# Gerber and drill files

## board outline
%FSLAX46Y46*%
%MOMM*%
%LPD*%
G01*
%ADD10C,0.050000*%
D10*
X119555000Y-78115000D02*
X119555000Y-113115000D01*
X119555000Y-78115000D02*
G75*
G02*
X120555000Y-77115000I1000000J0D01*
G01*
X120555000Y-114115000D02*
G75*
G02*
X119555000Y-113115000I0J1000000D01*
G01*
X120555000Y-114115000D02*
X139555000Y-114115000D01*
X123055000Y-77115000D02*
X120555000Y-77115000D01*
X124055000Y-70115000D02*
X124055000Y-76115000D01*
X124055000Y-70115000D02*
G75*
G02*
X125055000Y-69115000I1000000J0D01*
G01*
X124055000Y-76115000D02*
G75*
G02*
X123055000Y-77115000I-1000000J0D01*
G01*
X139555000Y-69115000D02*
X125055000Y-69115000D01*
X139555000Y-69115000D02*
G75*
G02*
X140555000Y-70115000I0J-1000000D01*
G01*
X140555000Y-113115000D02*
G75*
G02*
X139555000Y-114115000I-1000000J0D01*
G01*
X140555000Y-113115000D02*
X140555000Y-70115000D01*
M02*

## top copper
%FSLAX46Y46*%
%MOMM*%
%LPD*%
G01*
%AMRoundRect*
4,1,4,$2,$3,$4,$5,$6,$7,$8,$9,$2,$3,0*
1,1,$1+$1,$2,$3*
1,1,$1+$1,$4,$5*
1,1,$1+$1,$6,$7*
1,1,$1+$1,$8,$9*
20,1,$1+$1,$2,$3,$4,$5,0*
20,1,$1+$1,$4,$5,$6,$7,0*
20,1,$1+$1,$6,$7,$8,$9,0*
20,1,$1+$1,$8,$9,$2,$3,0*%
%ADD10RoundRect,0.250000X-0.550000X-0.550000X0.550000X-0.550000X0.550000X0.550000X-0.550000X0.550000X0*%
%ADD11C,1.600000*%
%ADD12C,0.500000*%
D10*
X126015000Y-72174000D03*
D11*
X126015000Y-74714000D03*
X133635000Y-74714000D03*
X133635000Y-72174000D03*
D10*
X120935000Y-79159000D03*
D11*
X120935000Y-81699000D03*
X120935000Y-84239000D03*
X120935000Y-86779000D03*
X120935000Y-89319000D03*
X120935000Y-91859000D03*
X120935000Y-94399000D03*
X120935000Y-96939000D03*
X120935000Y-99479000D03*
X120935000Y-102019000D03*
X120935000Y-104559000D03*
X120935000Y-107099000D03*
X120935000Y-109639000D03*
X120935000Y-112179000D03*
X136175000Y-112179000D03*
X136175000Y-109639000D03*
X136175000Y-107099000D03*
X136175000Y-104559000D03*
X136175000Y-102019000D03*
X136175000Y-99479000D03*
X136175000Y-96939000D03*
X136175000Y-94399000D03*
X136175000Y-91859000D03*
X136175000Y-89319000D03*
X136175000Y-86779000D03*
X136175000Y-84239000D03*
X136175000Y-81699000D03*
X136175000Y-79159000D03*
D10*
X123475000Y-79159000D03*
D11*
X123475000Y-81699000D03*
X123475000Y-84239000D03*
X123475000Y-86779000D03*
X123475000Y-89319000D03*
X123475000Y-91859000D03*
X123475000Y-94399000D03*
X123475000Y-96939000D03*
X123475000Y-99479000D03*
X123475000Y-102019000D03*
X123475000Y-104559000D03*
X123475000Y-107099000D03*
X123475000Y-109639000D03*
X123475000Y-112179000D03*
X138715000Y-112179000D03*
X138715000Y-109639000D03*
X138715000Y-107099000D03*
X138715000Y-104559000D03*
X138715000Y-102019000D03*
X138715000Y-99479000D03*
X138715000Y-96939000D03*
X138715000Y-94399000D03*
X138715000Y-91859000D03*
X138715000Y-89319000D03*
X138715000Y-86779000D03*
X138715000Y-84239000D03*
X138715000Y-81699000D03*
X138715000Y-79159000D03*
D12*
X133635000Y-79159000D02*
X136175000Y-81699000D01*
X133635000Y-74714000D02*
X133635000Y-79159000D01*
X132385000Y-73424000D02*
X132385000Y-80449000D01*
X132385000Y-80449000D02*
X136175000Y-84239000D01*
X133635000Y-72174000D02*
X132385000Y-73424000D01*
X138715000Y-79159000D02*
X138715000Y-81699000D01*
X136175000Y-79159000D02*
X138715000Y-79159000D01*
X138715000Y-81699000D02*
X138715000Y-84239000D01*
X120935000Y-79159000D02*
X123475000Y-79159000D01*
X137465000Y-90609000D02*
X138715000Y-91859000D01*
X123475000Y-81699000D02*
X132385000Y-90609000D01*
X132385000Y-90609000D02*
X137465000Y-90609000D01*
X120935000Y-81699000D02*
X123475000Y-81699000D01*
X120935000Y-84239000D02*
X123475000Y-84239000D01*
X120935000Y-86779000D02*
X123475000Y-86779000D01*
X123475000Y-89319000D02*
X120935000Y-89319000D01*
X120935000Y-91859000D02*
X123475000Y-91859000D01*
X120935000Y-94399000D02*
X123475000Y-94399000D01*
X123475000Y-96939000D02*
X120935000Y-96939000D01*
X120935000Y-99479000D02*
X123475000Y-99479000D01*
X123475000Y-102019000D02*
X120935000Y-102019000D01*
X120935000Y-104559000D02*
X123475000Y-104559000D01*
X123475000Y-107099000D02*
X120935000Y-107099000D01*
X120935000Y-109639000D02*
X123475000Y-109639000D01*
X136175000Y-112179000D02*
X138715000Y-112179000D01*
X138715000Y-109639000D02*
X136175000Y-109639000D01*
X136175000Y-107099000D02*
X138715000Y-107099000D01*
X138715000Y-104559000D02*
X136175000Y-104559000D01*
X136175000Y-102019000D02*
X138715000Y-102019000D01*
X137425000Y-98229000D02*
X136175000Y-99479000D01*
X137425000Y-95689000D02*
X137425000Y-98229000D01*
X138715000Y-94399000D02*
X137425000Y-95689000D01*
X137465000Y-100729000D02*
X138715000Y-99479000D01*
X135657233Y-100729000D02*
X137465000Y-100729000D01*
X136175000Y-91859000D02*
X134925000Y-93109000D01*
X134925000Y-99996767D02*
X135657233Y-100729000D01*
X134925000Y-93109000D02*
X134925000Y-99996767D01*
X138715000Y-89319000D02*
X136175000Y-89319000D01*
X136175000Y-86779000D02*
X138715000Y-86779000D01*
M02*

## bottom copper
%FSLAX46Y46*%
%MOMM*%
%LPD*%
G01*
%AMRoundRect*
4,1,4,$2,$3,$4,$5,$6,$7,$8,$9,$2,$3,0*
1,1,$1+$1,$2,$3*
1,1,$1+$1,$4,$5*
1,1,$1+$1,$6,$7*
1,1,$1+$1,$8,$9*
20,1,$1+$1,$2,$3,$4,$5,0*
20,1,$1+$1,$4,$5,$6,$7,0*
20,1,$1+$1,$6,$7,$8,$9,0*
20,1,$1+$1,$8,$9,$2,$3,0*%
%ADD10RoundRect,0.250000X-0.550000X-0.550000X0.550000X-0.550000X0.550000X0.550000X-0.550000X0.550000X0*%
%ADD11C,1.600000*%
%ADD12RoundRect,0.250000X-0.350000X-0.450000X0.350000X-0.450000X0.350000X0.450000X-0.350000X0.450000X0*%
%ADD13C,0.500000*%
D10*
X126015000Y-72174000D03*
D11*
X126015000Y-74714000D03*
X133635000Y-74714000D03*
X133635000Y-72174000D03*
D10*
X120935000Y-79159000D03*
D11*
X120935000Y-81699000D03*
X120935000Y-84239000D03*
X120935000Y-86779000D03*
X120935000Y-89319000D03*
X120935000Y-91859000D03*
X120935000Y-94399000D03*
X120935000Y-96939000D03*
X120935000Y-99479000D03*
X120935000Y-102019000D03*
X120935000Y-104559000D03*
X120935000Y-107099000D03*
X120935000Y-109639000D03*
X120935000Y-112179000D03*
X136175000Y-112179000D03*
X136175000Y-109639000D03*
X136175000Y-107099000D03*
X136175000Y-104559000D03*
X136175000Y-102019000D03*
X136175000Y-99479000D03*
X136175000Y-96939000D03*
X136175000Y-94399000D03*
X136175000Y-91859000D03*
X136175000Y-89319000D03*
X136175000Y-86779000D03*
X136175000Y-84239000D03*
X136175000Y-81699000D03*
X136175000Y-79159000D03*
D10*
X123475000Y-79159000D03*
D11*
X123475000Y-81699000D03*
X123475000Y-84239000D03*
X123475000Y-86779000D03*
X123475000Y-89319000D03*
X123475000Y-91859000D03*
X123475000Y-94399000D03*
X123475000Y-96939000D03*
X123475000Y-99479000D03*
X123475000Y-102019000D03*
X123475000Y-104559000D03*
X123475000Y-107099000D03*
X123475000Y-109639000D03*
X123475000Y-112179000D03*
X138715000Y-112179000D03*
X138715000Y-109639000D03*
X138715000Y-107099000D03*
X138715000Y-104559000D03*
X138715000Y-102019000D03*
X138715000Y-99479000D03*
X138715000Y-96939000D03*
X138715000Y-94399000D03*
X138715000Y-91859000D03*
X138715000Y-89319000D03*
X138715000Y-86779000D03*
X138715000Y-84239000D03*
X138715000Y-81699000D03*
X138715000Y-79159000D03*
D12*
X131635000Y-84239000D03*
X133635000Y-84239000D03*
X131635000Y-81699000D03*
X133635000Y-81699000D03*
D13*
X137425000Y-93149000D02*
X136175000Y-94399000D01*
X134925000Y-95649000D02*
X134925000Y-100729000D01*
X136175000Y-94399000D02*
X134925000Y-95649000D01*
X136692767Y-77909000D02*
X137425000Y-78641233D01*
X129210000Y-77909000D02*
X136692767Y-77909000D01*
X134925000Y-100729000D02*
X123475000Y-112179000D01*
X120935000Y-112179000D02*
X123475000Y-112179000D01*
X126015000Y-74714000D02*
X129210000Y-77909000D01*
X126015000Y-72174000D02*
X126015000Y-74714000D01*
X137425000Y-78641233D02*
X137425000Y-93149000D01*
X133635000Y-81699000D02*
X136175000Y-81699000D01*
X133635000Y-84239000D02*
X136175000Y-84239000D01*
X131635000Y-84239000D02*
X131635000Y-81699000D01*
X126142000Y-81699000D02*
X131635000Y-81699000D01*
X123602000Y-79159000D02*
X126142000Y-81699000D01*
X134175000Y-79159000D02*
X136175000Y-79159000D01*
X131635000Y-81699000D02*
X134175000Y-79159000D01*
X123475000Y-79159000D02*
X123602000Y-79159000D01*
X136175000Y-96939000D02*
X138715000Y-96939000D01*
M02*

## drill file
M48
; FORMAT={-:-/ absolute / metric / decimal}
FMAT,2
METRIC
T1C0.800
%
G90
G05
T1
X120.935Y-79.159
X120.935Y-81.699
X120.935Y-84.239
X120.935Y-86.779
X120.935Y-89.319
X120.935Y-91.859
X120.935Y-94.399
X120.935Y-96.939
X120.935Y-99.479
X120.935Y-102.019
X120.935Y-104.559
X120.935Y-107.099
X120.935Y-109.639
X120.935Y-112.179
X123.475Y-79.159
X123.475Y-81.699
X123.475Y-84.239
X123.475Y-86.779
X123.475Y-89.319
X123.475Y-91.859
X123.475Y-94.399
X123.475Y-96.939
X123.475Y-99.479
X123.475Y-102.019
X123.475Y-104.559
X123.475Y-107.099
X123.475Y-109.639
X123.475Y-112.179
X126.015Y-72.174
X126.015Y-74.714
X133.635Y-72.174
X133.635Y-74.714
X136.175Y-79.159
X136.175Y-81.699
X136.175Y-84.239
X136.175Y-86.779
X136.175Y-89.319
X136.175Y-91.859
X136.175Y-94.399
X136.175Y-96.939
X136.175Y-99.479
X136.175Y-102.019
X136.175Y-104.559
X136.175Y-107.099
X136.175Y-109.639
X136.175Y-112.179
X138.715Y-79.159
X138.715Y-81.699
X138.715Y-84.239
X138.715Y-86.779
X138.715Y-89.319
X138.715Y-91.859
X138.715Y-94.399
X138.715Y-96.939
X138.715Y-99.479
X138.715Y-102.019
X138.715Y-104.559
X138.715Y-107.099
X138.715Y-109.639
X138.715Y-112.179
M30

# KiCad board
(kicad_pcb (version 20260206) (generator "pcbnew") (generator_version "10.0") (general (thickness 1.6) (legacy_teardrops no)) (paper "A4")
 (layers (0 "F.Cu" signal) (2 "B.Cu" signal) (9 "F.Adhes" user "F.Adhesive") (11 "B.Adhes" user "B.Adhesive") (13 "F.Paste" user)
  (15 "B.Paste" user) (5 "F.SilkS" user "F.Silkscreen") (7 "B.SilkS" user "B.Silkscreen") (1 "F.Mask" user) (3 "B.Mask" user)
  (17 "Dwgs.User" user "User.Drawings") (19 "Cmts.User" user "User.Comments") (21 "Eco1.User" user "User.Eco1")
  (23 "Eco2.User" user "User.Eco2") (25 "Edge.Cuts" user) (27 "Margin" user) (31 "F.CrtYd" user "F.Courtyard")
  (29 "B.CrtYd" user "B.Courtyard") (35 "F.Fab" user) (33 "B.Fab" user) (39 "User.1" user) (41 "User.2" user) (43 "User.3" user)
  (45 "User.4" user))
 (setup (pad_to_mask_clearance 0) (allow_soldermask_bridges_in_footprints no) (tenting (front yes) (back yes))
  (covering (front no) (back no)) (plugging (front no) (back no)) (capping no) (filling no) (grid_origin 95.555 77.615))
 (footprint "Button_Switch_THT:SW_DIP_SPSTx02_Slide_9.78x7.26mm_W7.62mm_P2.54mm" (layer "F.Cu") (at 126.015 72.174)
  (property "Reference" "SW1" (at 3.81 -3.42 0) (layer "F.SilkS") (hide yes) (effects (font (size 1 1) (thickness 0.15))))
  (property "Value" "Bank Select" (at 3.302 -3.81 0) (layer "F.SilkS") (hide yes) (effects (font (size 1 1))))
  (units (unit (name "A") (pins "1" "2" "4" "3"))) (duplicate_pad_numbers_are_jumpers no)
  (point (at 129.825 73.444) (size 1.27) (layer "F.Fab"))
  (pad "1" thru_hole roundrect (at 0 0) (size 1.6 1.6) (drill 0.8) (layers "*.Cu" "*.Mask") (remove_unused_layers no)
   (roundrect_rratio 0.15625) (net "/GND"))
  (pad "2" thru_hole circle (at 0 2.54) (size 1.6 1.6) (drill 0.8) (layers "*.Cu" "*.Mask") (remove_unused_layers no) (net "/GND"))
  (pad "3" thru_hole circle (at 7.62 2.54) (size 1.6 1.6) (drill 0.8) (layers "*.Cu" "*.Mask") (remove_unused_layers no) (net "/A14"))
  (pad "4" thru_hole circle (at 7.62 0) (size 1.6 1.6) (drill 0.8) (layers "*.Cu" "*.Mask") (remove_unused_layers no) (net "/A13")))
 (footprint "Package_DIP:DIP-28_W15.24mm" (layer "F.Cu") (at 120.935 79.159)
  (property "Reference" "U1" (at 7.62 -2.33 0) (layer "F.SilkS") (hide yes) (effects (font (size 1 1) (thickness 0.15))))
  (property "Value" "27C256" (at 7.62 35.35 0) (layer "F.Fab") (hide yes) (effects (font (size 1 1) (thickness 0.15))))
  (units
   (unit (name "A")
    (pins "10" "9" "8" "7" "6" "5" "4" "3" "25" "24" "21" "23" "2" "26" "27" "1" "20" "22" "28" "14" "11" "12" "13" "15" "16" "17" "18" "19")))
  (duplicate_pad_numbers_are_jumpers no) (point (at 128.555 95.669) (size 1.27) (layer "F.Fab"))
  (pad "1" thru_hole roundrect (at 0 0) (size 1.6 1.6) (drill 0.8) (layers "*.Cu" "*.Mask") (remove_unused_layers no)
   (roundrect_rratio 0.15625) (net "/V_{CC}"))
  (pad "2" thru_hole circle (at 0 2.54) (size 1.6 1.6) (drill 0.8) (layers "*.Cu" "*.Mask") (remove_unused_layers no) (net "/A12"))
  (pad "3" thru_hole circle (at 0 5.08) (size 1.6 1.6) (drill 0.8) (layers "*.Cu" "*.Mask") (remove_unused_layers no) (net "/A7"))
  (pad "4" thru_hole circle (at 0 7.62) (size 1.6 1.6) (drill 0.8) (layers "*.Cu" "*.Mask") (remove_unused_layers no) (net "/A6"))
  (pad "5" thru_hole circle (at 0 10.16) (size 1.6 1.6) (drill 0.8) (layers "*.Cu" "*.Mask") (remove_unused_layers no) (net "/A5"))
  (pad "6" thru_hole circle (at 0 12.7) (size 1.6 1.6) (drill 0.8) (layers "*.Cu" "*.Mask") (remove_unused_layers no) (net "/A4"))
  (pad "7" thru_hole circle (at 0 15.24) (size 1.6 1.6) (drill 0.8) (layers "*.Cu" "*.Mask") (remove_unused_layers no) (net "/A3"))
  (pad "8" thru_hole circle (at 0 17.78) (size 1.6 1.6) (drill 0.8) (layers "*.Cu" "*.Mask") (remove_unused_layers no) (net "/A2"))
  (pad "9" thru_hole circle (at 0 20.32) (size 1.6 1.6) (drill 0.8) (layers "*.Cu" "*.Mask") (remove_unused_layers no) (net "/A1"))
  (pad "10" thru_hole circle (at 0 22.86) (size 1.6 1.6) (drill 0.8) (layers "*.Cu" "*.Mask") (remove_unused_layers no) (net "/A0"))
  (pad "11" thru_hole circle (at 0 25.4) (size 1.6 1.6) (drill 0.8) (layers "*.Cu" "*.Mask") (remove_unused_layers no) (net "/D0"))
  (pad "12" thru_hole circle (at 0 27.94) (size 1.6 1.6) (drill 0.8) (layers "*.Cu" "*.Mask") (remove_unused_layers no) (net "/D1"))
  (pad "13" thru_hole circle (at 0 30.48) (size 1.6 1.6) (drill 0.8) (layers "*.Cu" "*.Mask") (remove_unused_layers no) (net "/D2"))
  (pad "14" thru_hole circle (at 0 33.02) (size 1.6 1.6) (drill 0.8) (layers "*.Cu" "*.Mask") (remove_unused_layers no) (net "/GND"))
  (pad "15" thru_hole circle (at 15.24 33.02) (size 1.6 1.6) (drill 0.8) (layers "*.Cu" "*.Mask") (remove_unused_layers no) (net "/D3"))
  (pad "16" thru_hole circle (at 15.24 30.48) (size 1.6 1.6) (drill 0.8) (layers "*.Cu" "*.Mask") (remove_unused_layers no) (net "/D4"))
  (pad "17" thru_hole circle (at 15.24 27.94) (size 1.6 1.6) (drill 0.8) (layers "*.Cu" "*.Mask") (remove_unused_layers no) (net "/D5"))
  (pad "18" thru_hole circle (at 15.24 25.4) (size 1.6 1.6) (drill 0.8) (layers "*.Cu" "*.Mask") (remove_unused_layers no) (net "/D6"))
  (pad "19" thru_hole circle (at 15.24 22.86) (size 1.6 1.6) (drill 0.8) (layers "*.Cu" "*.Mask") (remove_unused_layers no) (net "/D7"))
  (pad "20" thru_hole circle (at 15.24 20.32) (size 1.6 1.6) (drill 0.8) (layers "*.Cu" "*.Mask") (remove_unused_layers no) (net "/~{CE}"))
  (pad "21" thru_hole circle (at 15.24 17.78) (size 1.6 1.6) (drill 0.8) (layers "*.Cu" "*.Mask") (remove_unused_layers no) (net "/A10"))
  (pad "22" thru_hole circle (at 15.24 15.24) (size 1.6 1.6) (drill 0.8) (layers "*.Cu" "*.Mask") (remove_unused_layers no) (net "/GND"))
  (pad "23" thru_hole circle (at 15.24 12.7) (size 1.6 1.6) (drill 0.8) (layers "*.Cu" "*.Mask") (remove_unused_layers no) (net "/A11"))
  (pad "24" thru_hole circle (at 15.24 10.16) (size 1.6 1.6) (drill 0.8) (layers "*.Cu" "*.Mask") (remove_unused_layers no) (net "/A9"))
  (pad "25" thru_hole circle (at 15.24 7.62) (size 1.6 1.6) (drill 0.8) (layers "*.Cu" "*.Mask") (remove_unused_layers no) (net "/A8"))
  (pad "26" thru_hole circle (at 15.24 5.08) (size 1.6 1.6) (drill 0.8) (layers "*.Cu" "*.Mask") (remove_unused_layers no) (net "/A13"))
  (pad "27" thru_hole circle (at 15.24 2.54) (size 1.6 1.6) (drill 0.8) (layers "*.Cu" "*.Mask") (remove_unused_layers no) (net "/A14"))
  (pad "28" thru_hole circle (at 15.24 0) (size 1.6 1.6) (drill 0.8) (layers "*.Cu" "*.Mask") (remove_unused_layers no) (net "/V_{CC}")))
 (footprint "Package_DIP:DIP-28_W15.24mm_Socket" (layer "F.Cu") (at 123.475 79.159)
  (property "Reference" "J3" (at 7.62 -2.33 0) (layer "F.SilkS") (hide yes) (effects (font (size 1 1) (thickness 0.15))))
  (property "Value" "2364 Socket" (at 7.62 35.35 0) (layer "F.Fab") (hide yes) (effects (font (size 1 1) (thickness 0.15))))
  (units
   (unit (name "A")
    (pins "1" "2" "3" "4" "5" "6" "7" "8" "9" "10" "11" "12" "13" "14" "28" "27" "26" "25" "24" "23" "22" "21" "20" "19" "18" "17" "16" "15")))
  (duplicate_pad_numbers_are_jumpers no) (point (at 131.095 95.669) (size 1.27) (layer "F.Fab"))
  (pad "1" thru_hole roundrect (at 0 0) (size 1.6 1.6) (drill 0.8) (layers "*.Cu" "*.Mask") (remove_unused_layers no)
   (roundrect_rratio 0.15625) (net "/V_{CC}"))
  (pad "2" thru_hole circle (at 0 2.54) (size 1.6 1.6) (drill 0.8) (layers "*.Cu" "*.Mask") (remove_unused_layers no) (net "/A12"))
  (pad "3" thru_hole circle (at 0 5.08) (size 1.6 1.6) (drill 0.8) (layers "*.Cu" "*.Mask") (remove_unused_layers no) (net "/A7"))
  (pad "4" thru_hole circle (at 0 7.62) (size 1.6 1.6) (drill 0.8) (layers "*.Cu" "*.Mask") (remove_unused_layers no) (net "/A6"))
  (pad "5" thru_hole circle (at 0 10.16) (size 1.6 1.6) (drill 0.8) (layers "*.Cu" "*.Mask") (remove_unused_layers no) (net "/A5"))
  (pad "6" thru_hole circle (at 0 12.7) (size 1.6 1.6) (drill 0.8) (layers "*.Cu" "*.Mask") (remove_unused_layers no) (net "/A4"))
  (pad "7" thru_hole circle (at 0 15.24) (size 1.6 1.6) (drill 0.8) (layers "*.Cu" "*.Mask") (remove_unused_layers no) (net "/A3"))
  (pad "8" thru_hole circle (at 0 17.78) (size 1.6 1.6) (drill 0.8) (layers "*.Cu" "*.Mask") (remove_unused_layers no) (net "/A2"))
  (pad "9" thru_hole circle (at 0 20.32) (size 1.6 1.6) (drill 0.8) (layers "*.Cu" "*.Mask") (remove_unused_layers no) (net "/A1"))
  (pad "10" thru_hole circle (at 0 22.86) (size 1.6 1.6) (drill 0.8) (layers "*.Cu" "*.Mask") (remove_unused_layers no) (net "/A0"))
  (pad "11" thru_hole circle (at 0 25.4) (size 1.6 1.6) (drill 0.8) (layers "*.Cu" "*.Mask") (remove_unused_layers no) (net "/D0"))
  (pad "12" thru_hole circle (at 0 27.94) (size 1.6 1.6) (drill 0.8) (layers "*.Cu" "*.Mask") (remove_unused_layers no) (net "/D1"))
  (pad "13" thru_hole circle (at 0 30.48) (size 1.6 1.6) (drill 0.8) (layers "*.Cu" "*.Mask") (remove_unused_layers no) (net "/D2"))
  (pad "14" thru_hole circle (at 0 33.02) (size 1.6 1.6) (drill 0.8) (layers "*.Cu" "*.Mask") (remove_unused_layers no) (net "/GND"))
  (pad "15" thru_hole circle (at 15.24 33.02) (size 1.6 1.6) (drill 0.8) (layers "*.Cu" "*.Mask") (remove_unused_layers no) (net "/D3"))
  (pad "16" thru_hole circle (at 15.24 30.48) (size 1.6 1.6) (drill 0.8) (layers "*.Cu" "*.Mask") (remove_unused_layers no) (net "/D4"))
  (pad "17" thru_hole circle (at 15.24 27.94) (size 1.6 1.6) (drill 0.8) (layers "*.Cu" "*.Mask") (remove_unused_layers no) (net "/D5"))
  (pad "18" thru_hole circle (at 15.24 25.4) (size 1.6 1.6) (drill 0.8) (layers "*.Cu" "*.Mask") (remove_unused_layers no) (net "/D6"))
  (pad "19" thru_hole circle (at 15.24 22.86) (size 1.6 1.6) (drill 0.8) (layers "*.Cu" "*.Mask") (remove_unused_layers no) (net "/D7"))
  (pad "20" thru_hole circle (at 15.24 20.32) (size 1.6 1.6) (drill 0.8) (layers "*.Cu" "*.Mask") (remove_unused_layers no) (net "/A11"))
  (pad "21" thru_hole circle (at 15.24 17.78) (size 1.6 1.6) (drill 0.8) (layers "*.Cu" "*.Mask") (remove_unused_layers no) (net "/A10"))
  (pad "22" thru_hole circle (at 15.24 15.24) (size 1.6 1.6) (drill 0.8) (layers "*.Cu" "*.Mask") (remove_unused_layers no) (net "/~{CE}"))
  (pad "23" thru_hole circle (at 15.24 12.7) (size 1.6 1.6) (drill 0.8) (layers "*.Cu" "*.Mask") (remove_unused_layers no) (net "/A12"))
  (pad "24" thru_hole circle (at 15.24 10.16) (size 1.6 1.6) (drill 0.8) (layers "*.Cu" "*.Mask") (remove_unused_layers no) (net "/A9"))
  (pad "25" thru_hole circle (at 15.24 7.62) (size 1.6 1.6) (drill 0.8) (layers "*.Cu" "*.Mask") (remove_unused_layers no) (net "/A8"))
  (pad "26" thru_hole circle (at 15.24 5.08) (size 1.6 1.6) (drill 0.8) (layers "*.Cu" "*.Mask") (remove_unused_layers no) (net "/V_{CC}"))
  (pad "27" thru_hole circle (at 15.24 2.54) (size 1.6 1.6) (drill 0.8) (layers "*.Cu" "*.Mask") (remove_unused_layers no) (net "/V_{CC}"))
  (pad "28" thru_hole circle (at 15.24 0) (size 1.6 1.6) (drill 0.8) (layers "*.Cu" "*.Mask") (remove_unused_layers no) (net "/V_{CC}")))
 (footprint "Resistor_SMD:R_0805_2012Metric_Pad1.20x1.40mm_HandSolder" (layer "B.Cu") (at 132.635 84.239)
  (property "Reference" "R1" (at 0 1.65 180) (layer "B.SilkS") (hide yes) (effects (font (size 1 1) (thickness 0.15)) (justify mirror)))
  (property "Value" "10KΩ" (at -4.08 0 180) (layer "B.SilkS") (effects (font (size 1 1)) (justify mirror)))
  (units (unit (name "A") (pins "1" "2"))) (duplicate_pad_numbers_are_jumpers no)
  (pad "1" smd roundrect (at -1 0) (size 1.2 1.4) (layers "B.Cu" "B.Mask" "B.Paste") (roundrect_rratio 0.208333) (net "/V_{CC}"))
  (pad "2" smd roundrect (at 1 0) (size 1.2 1.4) (layers "B.Cu" "B.Mask" "B.Paste") (roundrect_rratio 0.208333) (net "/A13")))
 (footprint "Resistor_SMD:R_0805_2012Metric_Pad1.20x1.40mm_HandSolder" (layer "B.Cu") (at 132.635 81.699)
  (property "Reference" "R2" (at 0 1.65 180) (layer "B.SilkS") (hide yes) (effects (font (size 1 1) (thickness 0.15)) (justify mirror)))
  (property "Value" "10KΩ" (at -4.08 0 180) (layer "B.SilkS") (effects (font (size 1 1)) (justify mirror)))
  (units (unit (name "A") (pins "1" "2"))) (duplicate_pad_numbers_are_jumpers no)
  (pad "1" smd roundrect (at -1 0) (size 1.2 1.4) (layers "B.Cu" "B.Mask" "B.Paste") (roundrect_rratio 0.208333) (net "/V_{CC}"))
  (pad "2" smd roundrect (at 1 0) (size 1.2 1.4) (layers "B.Cu" "B.Mask" "B.Paste") (roundrect_rratio 0.208333) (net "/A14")))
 (gr_line (start 119.555 78.115) (end 119.555 113.115) (stroke (width 0.05) (type default)) (layer "Edge.Cuts"))
 (gr_arc (start 119.555 78.115) (mid 119.847893 77.407893) (end 120.555 77.115) (stroke (width 0.05) (type default)) (layer "Edge.Cuts"))
 (gr_arc (start 120.555 114.115) (mid 119.847893 113.822107) (end 119.555 113.115) (stroke (width 0.05) (type default)) (layer "Edge.Cuts"))
 (gr_line (start 120.555 114.115) (end 139.555 114.115) (stroke (width 0.05) (type default)) (layer "Edge.Cuts"))
 (gr_line (start 123.055 77.115) (end 120.555 77.115) (stroke (width 0.05) (type default)) (layer "Edge.Cuts"))
 (gr_line (start 124.055 70.115) (end 124.055 76.115) (stroke (width 0.05) (type default)) (layer "Edge.Cuts"))
 (gr_arc (start 124.055 70.115) (mid 124.347893 69.407893) (end 125.055 69.115) (stroke (width 0.05) (type default)) (layer "Edge.Cuts"))
 (gr_arc (start 124.055 76.115) (mid 123.762107 76.822107) (end 123.055 77.115) (stroke (width 0.05) (type default)) (layer "Edge.Cuts"))
 (gr_line (start 139.555 69.115) (end 125.055 69.115) (stroke (width 0.05) (type default)) (layer "Edge.Cuts"))
 (gr_arc (start 139.555 69.115) (mid 140.262107 69.407893) (end 140.555 70.115) (stroke (width 0.05) (type default)) (layer "Edge.Cuts"))
 (gr_arc (start 140.555 113.115) (mid 140.262107 113.822107) (end 139.555 114.115) (stroke (width 0.05) (type default)) (layer "Edge.Cuts"))
 (gr_line (start 140.555 113.115) (end 140.555 70.115) (stroke (width 0.05) (type default)) (layer "Edge.Cuts"))
 (segment (start 137.425 93.149) (end 136.175 94.399) (width 0.5) (layer "B.Cu") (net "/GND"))
 (segment (start 134.925 95.649) (end 134.925 100.729) (width 0.5) (layer "B.Cu") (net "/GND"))
 (segment (start 136.175 94.399) (end 134.925 95.649) (width 0.5) (layer "B.Cu") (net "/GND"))
 (segment (start 136.692767 77.909) (end 137.425 78.641233) (width 0.5) (layer "B.Cu") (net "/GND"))
 (segment (start 129.21 77.909) (end 136.692767 77.909) (width 0.5) (layer "B.Cu") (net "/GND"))
 (segment (start 134.925 100.729) (end 123.475 112.179) (width 0.5) (layer "B.Cu") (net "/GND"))
 (segment (start 120.935 112.179) (end 123.475 112.179) (width 0.5) (layer "B.Cu") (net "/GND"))
 (segment (start 126.015 74.714) (end 129.21 77.909) (width 0.5) (layer "B.Cu") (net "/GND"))
 (segment (start 126.015 72.174) (end 126.015 74.714) (width 0.5) (layer "B.Cu") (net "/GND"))
 (segment (start 137.425 78.641233) (end 137.425 93.149) (width 0.5) (layer "B.Cu") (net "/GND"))
 (segment (start 133.635 79.159) (end 136.175 81.699) (width 0.5) (layer "F.Cu") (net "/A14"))
 (segment (start 133.635 74.714) (end 133.635 79.159) (width 0.5) (layer "F.Cu") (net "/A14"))
 (segment (start 133.635 81.699) (end 136.175 81.699) (width 0.5) (layer "B.Cu") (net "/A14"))
 (segment (start 132.385 73.424) (end 132.385 80.449) (width 0.5) (layer "F.Cu") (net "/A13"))
 (segment (start 132.385 80.449) (end 136.175 84.239) (width 0.5) (layer "F.Cu") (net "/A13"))
 (segment (start 133.635 72.174) (end 132.385 73.424) (width 0.5) (layer "F.Cu") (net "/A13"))
 (segment (start 133.635 84.239) (end 136.175 84.239) (width 0.5) (layer "B.Cu") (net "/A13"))
 (segment (start 138.715 79.159) (end 138.715 81.699) (width 0.5) (layer "F.Cu") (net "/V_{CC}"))
 (segment (start 136.175 79.159) (end 138.715 79.159) (width 0.5) (layer "F.Cu") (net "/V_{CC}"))
 (segment (start 138.715 81.699) (end 138.715 84.239) (width 0.5) (layer "F.Cu") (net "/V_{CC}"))
 (segment (start 120.935 79.159) (end 123.475 79.159) (width 0.5) (layer "F.Cu") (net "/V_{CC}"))
 (segment (start 131.635 84.239) (end 131.635 81.699) (width 0.5) (layer "B.Cu") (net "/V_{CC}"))
 (segment (start 126.142 81.699) (end 131.635 81.699) (width 0.5) (layer "B.Cu") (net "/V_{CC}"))
 (segment (start 123.602 79.159) (end 126.142 81.699) (width 0.5) (layer "B.Cu") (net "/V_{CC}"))
 (segment (start 134.175 79.159) (end 136.175 79.159) (width 0.5) (layer "B.Cu") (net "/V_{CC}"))
 (segment (start 131.635 81.699) (end 134.175 79.159) (width 0.5) (layer "B.Cu") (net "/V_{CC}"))
 (segment (start 123.475 79.159) (end 123.602 79.159) (width 0.5) (layer "B.Cu") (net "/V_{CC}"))
 (segment (start 137.465 90.609) (end 138.715 91.859) (width 0.5) (layer "F.Cu") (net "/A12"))
 (segment (start 123.475 81.699) (end 132.385 90.609) (width 0.5) (layer "F.Cu") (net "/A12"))
 (segment (start 132.385 90.609) (end 137.465 90.609) (width 0.5) (layer "F.Cu") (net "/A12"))
 (segment (start 120.935 81.699) (end 123.475 81.699) (width 0.5) (layer "F.Cu") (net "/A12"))
 (segment (start 120.935 84.239) (end 123.475 84.239) (width 0.5) (layer "F.Cu") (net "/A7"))
 (segment (start 120.935 86.779) (end 123.475 86.779) (width 0.5) (layer "F.Cu") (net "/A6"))
 (segment (start 123.475 89.319) (end 120.935 89.319) (width 0.5) (layer "F.Cu") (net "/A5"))
 (segment (start 120.935 91.859) (end 123.475 91.859) (width 0.5) (layer "F.Cu") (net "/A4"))
 (segment (start 120.935 94.399) (end 123.475 94.399) (width 0.5) (layer "F.Cu") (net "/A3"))
 (segment (start 123.475 96.939) (end 120.935 96.939) (width 0.5) (layer "F.Cu") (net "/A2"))
 (segment (start 120.935 99.479) (end 123.475 99.479) (width 0.5) (layer "F.Cu") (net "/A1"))
 (segment (start 123.475 102.019) (end 120.935 102.019) (width 0.5) (layer "F.Cu") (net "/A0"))
 (segment (start 120.935 104.559) (end 123.475 104.559) (width 0.5) (layer "F.Cu") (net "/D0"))
 (segment (start 123.475 107.099) (end 120.935 107.099) (width 0.5) (layer "F.Cu") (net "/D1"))
 (segment (start 120.935 109.639) (end 123.475 109.639) (width 0.5) (layer "F.Cu") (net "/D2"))
 (segment (start 136.175 112.179) (end 138.715 112.179) (width 0.5) (layer "F.Cu") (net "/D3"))
 (segment (start 138.715 109.639) (end 136.175 109.639) (width 0.5) (layer "F.Cu") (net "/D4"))
 (segment (start 136.175 107.099) (end 138.715 107.099) (width 0.5) (layer "F.Cu") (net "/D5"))
 (segment (start 138.715 104.559) (end 136.175 104.559) (width 0.5) (layer "F.Cu") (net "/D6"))
 (segment (start 136.175 102.019) (end 138.715 102.019) (width 0.5) (layer "F.Cu") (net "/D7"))
 (segment (start 137.425 98.229) (end 136.175 99.479) (width 0.5) (layer "F.Cu") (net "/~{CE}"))
 (segment (start 137.425 95.689) (end 137.425 98.229) (width 0.5) (layer "F.Cu") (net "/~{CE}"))
 (segment (start 138.715 94.399) (end 137.425 95.689) (width 0.5) (layer "F.Cu") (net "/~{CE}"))
 (segment (start 136.175 96.939) (end 138.715 96.939) (width 0.5) (layer "B.Cu") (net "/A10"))
 (segment (start 137.465 100.729) (end 138.715 99.479) (width 0.5) (layer "F.Cu") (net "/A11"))
 (segment (start 135.657233 100.729) (end 137.465 100.729) (width 0.5) (layer "F.Cu") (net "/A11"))
 (segment (start 136.175 91.859) (end 134.925 93.109) (width 0.5) (layer "F.Cu") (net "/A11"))
 (segment (start 134.925 99.996767) (end 135.657233 100.729) (width 0.5) (layer "F.Cu") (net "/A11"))
 (segment (start 134.925 93.109) (end 134.925 99.996767) (width 0.5) (layer "F.Cu") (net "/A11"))
 (segment (start 138.715 89.319) (end 136.175 89.319) (width 0.5) (layer "F.Cu") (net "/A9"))
 (segment (start 136.175 86.779) (end 138.715 86.779) (width 0.5) (layer "F.Cu") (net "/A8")))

